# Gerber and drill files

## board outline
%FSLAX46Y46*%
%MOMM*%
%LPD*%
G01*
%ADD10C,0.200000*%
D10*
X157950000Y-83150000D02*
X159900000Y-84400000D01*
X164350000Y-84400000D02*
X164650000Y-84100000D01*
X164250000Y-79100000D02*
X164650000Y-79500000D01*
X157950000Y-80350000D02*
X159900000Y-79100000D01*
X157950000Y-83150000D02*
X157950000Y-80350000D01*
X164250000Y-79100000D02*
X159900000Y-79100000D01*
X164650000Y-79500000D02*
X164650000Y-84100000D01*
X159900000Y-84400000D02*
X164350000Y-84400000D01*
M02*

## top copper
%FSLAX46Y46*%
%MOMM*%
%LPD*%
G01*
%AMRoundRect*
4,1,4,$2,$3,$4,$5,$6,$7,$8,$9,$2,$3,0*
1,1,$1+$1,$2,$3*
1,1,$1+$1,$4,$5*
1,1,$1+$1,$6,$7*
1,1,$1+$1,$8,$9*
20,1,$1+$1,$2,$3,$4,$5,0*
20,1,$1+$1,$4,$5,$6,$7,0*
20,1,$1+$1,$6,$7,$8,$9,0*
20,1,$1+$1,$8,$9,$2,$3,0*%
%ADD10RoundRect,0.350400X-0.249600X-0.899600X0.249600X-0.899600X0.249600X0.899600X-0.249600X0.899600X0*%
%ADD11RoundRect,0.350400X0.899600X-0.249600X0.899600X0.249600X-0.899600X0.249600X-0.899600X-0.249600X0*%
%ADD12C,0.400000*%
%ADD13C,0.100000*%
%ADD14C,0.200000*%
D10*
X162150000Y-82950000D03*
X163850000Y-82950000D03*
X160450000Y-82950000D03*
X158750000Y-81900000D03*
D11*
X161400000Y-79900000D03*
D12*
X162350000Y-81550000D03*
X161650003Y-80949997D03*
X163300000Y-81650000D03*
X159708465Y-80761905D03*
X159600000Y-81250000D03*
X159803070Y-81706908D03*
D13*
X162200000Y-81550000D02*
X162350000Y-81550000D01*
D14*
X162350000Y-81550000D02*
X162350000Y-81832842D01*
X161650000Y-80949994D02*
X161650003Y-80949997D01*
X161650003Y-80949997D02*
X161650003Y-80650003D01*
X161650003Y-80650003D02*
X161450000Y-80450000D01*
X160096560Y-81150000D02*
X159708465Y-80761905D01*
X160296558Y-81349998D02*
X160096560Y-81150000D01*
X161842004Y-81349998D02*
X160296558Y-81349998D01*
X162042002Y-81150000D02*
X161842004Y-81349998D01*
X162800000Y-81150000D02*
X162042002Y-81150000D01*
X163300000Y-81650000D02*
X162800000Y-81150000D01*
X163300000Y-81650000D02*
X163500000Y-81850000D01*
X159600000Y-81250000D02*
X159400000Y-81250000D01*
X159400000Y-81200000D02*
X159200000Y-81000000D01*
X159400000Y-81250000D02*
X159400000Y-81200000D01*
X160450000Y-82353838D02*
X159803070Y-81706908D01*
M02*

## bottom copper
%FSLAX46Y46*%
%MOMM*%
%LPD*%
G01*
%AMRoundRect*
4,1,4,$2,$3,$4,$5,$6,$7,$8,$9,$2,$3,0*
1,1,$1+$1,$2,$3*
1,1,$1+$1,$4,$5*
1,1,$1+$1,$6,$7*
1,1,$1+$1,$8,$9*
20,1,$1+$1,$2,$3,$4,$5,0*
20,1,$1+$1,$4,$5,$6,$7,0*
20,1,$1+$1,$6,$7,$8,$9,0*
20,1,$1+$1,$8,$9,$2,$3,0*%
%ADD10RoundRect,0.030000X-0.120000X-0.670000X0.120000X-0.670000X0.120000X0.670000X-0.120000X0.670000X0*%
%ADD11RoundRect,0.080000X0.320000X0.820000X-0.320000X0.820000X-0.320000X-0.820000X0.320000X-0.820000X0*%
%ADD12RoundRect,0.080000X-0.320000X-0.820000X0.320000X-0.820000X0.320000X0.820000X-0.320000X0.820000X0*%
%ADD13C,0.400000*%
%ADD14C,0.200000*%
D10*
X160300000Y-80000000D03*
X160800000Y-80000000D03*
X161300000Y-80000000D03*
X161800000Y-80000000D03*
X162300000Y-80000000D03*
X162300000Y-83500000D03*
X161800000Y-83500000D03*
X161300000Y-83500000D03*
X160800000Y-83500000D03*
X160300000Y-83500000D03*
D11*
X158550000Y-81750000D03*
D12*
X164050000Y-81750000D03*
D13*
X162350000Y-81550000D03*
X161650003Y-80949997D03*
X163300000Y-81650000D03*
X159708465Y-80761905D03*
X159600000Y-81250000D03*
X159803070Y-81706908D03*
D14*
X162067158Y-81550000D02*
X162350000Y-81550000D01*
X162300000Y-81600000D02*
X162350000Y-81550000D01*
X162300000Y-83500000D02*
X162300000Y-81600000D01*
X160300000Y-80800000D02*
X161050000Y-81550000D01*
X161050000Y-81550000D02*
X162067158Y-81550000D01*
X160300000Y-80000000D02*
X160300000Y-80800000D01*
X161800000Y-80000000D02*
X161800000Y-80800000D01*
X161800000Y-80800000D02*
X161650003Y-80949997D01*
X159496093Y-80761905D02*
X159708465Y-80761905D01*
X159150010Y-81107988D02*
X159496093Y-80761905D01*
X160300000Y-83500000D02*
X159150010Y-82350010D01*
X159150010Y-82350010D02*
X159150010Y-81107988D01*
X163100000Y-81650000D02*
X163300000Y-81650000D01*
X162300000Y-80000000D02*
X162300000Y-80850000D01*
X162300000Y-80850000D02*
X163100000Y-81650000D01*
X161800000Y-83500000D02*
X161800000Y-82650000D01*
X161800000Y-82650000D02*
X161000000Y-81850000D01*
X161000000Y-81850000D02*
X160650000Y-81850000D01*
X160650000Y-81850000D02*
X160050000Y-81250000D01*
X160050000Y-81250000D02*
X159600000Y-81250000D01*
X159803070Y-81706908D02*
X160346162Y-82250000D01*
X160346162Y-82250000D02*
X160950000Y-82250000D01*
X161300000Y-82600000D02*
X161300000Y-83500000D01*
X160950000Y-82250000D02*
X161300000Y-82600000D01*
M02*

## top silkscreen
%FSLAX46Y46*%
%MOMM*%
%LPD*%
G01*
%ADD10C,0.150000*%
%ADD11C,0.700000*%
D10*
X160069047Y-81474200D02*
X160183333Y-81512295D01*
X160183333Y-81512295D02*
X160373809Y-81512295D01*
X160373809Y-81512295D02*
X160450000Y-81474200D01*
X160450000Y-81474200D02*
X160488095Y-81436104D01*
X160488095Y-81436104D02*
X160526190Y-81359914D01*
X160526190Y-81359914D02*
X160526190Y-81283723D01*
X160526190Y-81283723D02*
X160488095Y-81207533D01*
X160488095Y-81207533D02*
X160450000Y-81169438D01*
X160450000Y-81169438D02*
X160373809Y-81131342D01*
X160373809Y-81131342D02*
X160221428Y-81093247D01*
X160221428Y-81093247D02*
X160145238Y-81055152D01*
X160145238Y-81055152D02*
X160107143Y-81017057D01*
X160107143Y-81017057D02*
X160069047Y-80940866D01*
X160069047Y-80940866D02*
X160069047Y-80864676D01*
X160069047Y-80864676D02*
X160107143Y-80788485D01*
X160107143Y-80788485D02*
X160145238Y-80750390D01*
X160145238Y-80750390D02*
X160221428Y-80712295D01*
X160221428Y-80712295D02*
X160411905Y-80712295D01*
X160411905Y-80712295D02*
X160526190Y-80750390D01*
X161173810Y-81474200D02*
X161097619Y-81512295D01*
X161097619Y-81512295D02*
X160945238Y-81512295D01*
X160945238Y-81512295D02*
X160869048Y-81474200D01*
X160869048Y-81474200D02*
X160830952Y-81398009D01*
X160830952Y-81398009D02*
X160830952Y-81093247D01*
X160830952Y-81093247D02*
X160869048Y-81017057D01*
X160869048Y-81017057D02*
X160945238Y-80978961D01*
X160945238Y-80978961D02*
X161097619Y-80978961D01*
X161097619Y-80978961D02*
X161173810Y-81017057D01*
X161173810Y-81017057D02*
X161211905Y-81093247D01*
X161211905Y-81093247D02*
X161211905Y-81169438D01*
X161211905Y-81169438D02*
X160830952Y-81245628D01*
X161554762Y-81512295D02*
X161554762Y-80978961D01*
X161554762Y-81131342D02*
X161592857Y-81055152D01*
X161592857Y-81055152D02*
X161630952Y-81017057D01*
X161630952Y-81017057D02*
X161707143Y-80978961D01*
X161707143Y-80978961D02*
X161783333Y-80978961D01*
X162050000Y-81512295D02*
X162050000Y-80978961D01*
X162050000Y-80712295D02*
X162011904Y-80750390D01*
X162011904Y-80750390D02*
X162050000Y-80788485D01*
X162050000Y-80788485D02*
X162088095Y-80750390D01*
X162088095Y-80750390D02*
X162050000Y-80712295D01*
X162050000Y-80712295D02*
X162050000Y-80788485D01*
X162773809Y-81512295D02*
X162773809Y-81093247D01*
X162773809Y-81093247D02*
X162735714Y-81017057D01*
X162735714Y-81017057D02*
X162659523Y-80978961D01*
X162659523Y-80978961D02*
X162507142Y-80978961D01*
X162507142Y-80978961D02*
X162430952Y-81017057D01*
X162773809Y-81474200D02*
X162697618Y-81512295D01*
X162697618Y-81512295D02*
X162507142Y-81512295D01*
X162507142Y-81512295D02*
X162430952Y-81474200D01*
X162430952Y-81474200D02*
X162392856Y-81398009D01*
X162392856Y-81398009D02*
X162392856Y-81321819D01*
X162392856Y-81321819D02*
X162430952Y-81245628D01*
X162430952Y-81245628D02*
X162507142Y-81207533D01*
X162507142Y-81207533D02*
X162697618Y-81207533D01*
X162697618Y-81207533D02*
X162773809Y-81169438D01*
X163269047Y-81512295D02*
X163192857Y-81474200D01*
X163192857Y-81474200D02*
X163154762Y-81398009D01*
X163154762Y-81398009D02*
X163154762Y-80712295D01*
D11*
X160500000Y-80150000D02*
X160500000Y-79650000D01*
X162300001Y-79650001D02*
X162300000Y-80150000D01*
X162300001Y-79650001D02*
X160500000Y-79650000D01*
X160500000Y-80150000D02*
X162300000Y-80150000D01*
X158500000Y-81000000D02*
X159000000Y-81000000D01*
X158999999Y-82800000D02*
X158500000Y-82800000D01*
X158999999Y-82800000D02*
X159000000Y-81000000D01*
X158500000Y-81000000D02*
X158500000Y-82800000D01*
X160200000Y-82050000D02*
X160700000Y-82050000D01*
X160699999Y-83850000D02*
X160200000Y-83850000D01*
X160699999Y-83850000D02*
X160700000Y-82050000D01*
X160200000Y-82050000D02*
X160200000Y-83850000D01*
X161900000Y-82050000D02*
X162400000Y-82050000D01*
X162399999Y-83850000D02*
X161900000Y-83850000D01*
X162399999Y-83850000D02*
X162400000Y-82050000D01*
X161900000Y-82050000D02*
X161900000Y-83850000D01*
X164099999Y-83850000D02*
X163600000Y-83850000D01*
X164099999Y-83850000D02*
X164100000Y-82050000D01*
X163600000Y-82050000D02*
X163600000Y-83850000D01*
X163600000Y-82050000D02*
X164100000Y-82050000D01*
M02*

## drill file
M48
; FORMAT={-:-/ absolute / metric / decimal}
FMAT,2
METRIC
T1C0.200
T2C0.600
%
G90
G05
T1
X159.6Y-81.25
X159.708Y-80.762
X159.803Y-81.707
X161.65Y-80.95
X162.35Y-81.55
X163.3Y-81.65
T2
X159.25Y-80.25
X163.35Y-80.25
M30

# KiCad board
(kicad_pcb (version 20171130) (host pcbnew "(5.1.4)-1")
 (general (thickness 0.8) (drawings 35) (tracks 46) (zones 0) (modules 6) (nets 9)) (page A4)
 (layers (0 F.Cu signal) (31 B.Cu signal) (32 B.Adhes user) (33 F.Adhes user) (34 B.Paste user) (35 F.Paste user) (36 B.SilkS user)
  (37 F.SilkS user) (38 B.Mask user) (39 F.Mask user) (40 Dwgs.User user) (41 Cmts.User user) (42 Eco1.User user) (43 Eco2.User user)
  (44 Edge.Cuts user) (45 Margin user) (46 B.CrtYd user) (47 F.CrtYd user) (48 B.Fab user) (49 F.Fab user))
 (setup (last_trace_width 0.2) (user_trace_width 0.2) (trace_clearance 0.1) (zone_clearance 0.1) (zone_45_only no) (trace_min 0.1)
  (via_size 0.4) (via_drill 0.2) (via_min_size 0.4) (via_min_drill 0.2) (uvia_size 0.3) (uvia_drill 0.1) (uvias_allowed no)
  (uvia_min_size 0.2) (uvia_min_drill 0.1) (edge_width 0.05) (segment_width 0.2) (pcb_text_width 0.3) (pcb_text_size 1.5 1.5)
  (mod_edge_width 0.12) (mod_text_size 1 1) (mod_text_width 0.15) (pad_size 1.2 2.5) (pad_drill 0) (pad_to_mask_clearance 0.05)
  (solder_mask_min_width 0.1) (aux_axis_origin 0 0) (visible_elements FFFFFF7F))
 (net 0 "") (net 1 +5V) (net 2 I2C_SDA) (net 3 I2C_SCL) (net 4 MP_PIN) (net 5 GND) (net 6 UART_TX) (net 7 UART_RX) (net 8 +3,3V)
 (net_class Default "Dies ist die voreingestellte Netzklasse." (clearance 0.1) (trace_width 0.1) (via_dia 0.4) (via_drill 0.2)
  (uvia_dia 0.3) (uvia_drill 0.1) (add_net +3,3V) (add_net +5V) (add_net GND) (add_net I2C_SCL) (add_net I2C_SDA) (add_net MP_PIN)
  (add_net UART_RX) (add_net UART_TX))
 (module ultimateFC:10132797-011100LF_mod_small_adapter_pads (layer B.Cu) (at 161.3 81.75 180)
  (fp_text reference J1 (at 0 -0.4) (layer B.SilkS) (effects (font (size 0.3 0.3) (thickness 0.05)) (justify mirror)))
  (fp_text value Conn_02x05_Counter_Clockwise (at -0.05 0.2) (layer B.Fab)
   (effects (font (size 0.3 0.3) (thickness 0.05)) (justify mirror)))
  (pad 1 smd roundrect (at 1 1.75) (size 0.3 1.4) (layers B.Cu B.Paste B.Mask) (roundrect_rratio 0.1) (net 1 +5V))
  (pad 2 smd roundrect (at 0.5 1.75) (size 0.3 1.4) (layers B.Cu B.Paste B.Mask) (roundrect_rratio 0.1) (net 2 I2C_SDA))
  (pad 3 smd roundrect (at 0 1.75) (size 0.3 1.4) (layers B.Cu B.Paste B.Mask) (roundrect_rratio 0.1) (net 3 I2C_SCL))
  (pad 4 smd roundrect (at -0.5 1.75) (size 0.3 1.4) (layers B.Cu B.Paste B.Mask) (roundrect_rratio 0.1) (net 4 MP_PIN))
  (pad 5 smd roundrect (at -1 1.75) (size 0.3 1.4) (layers B.Cu B.Paste B.Mask) (roundrect_rratio 0.1) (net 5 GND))
  (pad 6 smd roundrect (at -1 -1.75) (size 0.3 1.4) (layers B.Cu B.Paste B.Mask) (roundrect_rratio 0.1) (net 1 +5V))
  (pad 7 smd roundrect (at -0.5 -1.75) (size 0.3 1.4) (layers B.Cu B.Paste B.Mask) (roundrect_rratio 0.1) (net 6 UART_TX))
  (pad 8 smd roundrect (at 0 -1.75) (size 0.3 1.4) (layers B.Cu B.Paste B.Mask) (roundrect_rratio 0.1) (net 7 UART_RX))
  (pad 9 smd roundrect (at 0.5 -1.75) (size 0.3 1.4) (layers B.Cu B.Paste B.Mask) (roundrect_rratio 0.1) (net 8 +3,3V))
  (pad 10 smd roundrect (at 1 -1.75) (size 0.3 1.4) (layers B.Cu B.Paste B.Mask) (roundrect_rratio 0.1) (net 5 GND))
  (pad "" smd roundrect (at 2.75 0 180) (size 0.8 1.8) (layers B.Cu B.Paste B.Mask) (roundrect_rratio 0.1))
  (pad "" smd roundrect (at -2.75 0) (size 0.8 1.8) (layers B.Cu B.Paste B.Mask) (roundrect_rratio 0.1))
  (pad "" np_thru_hole circle (at 2.05 1.5 180) (size 0.6 0.6) (drill 0.6) (layers *.Cu *.Mask) (solder_mask_margin -0.001))
  (pad "" np_thru_hole circle (at -2.05 1.5 180) (size 0.6 0.6) (drill 0.6) (layers *.Cu *.Mask) (solder_mask_margin -0.001)))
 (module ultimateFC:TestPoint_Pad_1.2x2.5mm (layer F.Cu) (at 162.15 82.95)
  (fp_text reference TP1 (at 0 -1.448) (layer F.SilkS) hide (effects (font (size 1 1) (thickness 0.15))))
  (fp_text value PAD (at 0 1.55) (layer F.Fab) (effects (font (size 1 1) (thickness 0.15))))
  (pad 1 smd roundrect (at 0 0) (size 1.2 2.5) (layers F.Cu F.Mask) (roundrect_rratio 0.292) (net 1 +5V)))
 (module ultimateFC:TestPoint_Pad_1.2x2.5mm (layer F.Cu) (at 163.85 82.95)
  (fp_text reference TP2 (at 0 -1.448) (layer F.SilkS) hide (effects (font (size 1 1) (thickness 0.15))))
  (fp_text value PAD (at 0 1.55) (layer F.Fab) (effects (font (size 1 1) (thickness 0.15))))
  (pad 1 smd roundrect (at 0 0) (size 1.2 2.5) (layers F.Cu F.Mask) (roundrect_rratio 0.292) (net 5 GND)))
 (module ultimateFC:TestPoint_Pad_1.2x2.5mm (layer F.Cu) (at 160.45 82.95)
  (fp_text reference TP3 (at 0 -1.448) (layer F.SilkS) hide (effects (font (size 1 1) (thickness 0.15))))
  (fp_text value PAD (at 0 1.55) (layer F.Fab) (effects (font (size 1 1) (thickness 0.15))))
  (pad 1 smd roundrect (at 0 0) (size 1.2 2.5) (layers F.Cu F.Mask) (roundrect_rratio 0.292) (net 7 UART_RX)))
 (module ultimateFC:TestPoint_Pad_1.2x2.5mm (layer F.Cu) (at 158.75 81.9)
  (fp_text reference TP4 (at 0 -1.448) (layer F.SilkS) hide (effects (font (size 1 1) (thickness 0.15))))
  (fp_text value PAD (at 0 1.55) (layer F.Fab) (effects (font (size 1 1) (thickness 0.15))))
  (pad 1 smd roundrect (at 0 0) (size 1.2 2.5) (layers F.Cu F.Mask) (roundrect_rratio 0.292) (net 6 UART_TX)))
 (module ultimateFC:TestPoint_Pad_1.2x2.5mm (layer F.Cu) (at 161.4 79.9 90)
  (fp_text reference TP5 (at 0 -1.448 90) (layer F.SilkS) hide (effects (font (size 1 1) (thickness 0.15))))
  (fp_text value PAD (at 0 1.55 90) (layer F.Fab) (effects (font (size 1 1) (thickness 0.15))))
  (pad 1 smd roundrect (at 0 0 90) (size 1.2 2.5) (layers F.Cu F.Mask) (roundrect_rratio 0.292) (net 4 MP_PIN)))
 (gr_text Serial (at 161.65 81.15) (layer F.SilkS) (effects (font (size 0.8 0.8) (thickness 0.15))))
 (gr_line (start 160.5 80.15) (end 160.5 79.65) (layer F.SilkS) (width 0.7))
 (gr_line (start 162.300001 79.650001) (end 162.3 80.15) (layer F.SilkS) (width 0.7))
 (gr_line (start 162.300001 79.650001) (end 160.5 79.65) (layer F.SilkS) (width 0.7))
 (gr_line (start 160.5 80.15) (end 162.3 80.15) (layer F.SilkS) (width 0.7))
 (gr_line (start 158.5 81) (end 159 81) (layer F.SilkS) (width 0.7))
 (gr_line (start 158.999999 82.8) (end 158.5 82.8) (layer F.SilkS) (width 0.7))
 (gr_line (start 158.999999 82.8) (end 159 81) (layer F.SilkS) (width 0.7))
 (gr_line (start 158.5 81) (end 158.5 82.8) (layer F.SilkS) (width 0.7))
 (gr_line (start 160.2 82.05) (end 160.7 82.05) (layer F.SilkS) (width 0.7))
 (gr_line (start 160.699999 83.85) (end 160.2 83.85) (layer F.SilkS) (width 0.7))
 (gr_line (start 160.699999 83.85) (end 160.7 82.05) (layer F.SilkS) (width 0.7))
 (gr_line (start 160.2 82.05) (end 160.2 83.85) (layer F.SilkS) (width 0.7))
 (gr_line (start 161.9 82.05) (end 162.4 82.05) (layer F.SilkS) (width 0.7))
 (gr_line (start 162.399999 83.85) (end 161.9 83.85) (layer F.SilkS) (width 0.7))
 (gr_line (start 162.399999 83.85) (end 162.4 82.05) (layer F.SilkS) (width 0.7))
 (gr_line (start 161.9 82.05) (end 161.9 83.85) (layer F.SilkS) (width 0.7))
 (gr_line (start 164.099999 83.85) (end 163.6 83.85) (layer F.SilkS) (width 0.7))
 (gr_line (start 164.099999 83.85) (end 164.1 82.05) (layer F.SilkS) (width 0.7))
 (gr_line (start 163.6 82.05) (end 163.6 83.85) (layer F.SilkS) (width 0.7))
 (gr_line (start 163.6 82.05) (end 164.1 82.05) (layer F.SilkS) (width 0.7))
 (gr_line (start 157.95 83.15) (end 159.9 84.4) (layer Edge.Cuts) (width 0.2))
 (gr_line (start 164.35 84.4) (end 164.65 84.1) (layer Edge.Cuts) (width 0.2))
 (gr_line (start 164.25 79.1) (end 164.65 79.5) (layer Edge.Cuts) (width 0.2))
 (gr_line (start 157.95 80.35) (end 159.9 79.1) (layer Edge.Cuts) (width 0.2))
 (gr_line (start 157.95 83.15) (end 157.95 80.35) (layer Edge.Cuts) (width 0.2))
 (gr_line (start 164.25 79.1) (end 159.9 79.1) (layer Edge.Cuts) (width 0.2))
 (gr_line (start 164.65 79.5) (end 164.65 84.1) (layer Edge.Cuts) (width 0.2))
 (gr_line (start 159.9 84.4) (end 164.35 84.4) (layer Edge.Cuts) (width 0.2))
 (segment (start 162.067158 81.55) (end 162.35 81.55) (width 0.2) (layer B.Cu) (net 1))
 (segment (start 162.3 81.6) (end 162.35 81.55) (width 0.2) (layer B.Cu) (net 1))
 (segment (start 162.3 83.5) (end 162.3 81.6) (width 0.2) (layer B.Cu) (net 1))
 (segment (start 162.2 81.55) (end 162.35 81.55) (width 0.1) (layer F.Cu) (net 1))
 (segment (start 160.3 80.8) (end 161.05 81.55) (width 0.2) (layer B.Cu) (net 1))
 (segment (start 161.05 81.55) (end 162.067158 81.55) (width 0.2) (layer B.Cu) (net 1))
 (segment (start 160.3 80) (end 160.3 80.8) (width 0.2) (layer B.Cu) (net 1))
 (via (at 162.35 81.55) (size 0.4) (drill 0.2) (layers F.Cu B.Cu) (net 1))
 (segment (start 162.35 81.55) (end 162.35 81.832842) (width 0.2) (layer F.Cu) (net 1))
 (via (at 161.650003 80.949997) (size 0.4) (drill 0.2) (layers F.Cu B.Cu) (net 4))
 (segment (start 161.8 80) (end 161.8 80.8) (width 0.2) (layer B.Cu) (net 4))
 (segment (start 161.8 80.8) (end 161.650003 80.949997) (width 0.2) (layer B.Cu) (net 4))
 (segment (start 161.65 80.949994) (end 161.650003 80.949997) (width 0.2) (layer F.Cu) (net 4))
 (segment (start 161.650003 80.949997) (end 161.650003 80.650003) (width 0.2) (layer F.Cu) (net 4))
 (segment (start 161.650003 80.650003) (end 161.45 80.45) (width 0.2) (layer F.Cu) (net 4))
 (via (at 163.3 81.65) (size 0.4) (drill 0.2) (layers F.Cu B.Cu) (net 5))
 (via (at 159.708465 80.761905) (size 0.4) (drill 0.2) (layers F.Cu B.Cu) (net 5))
 (segment (start 159.496093 80.761905) (end 159.708465 80.761905) (width 0.2) (layer B.Cu) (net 5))
 (segment (start 159.15001 81.107988) (end 159.496093 80.761905) (width 0.2) (layer B.Cu) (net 5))
 (segment (start 160.3 83.5) (end 159.15001 82.35001) (width 0.2) (layer B.Cu) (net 5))
 (segment (start 159.15001 82.35001) (end 159.15001 81.107988) (width 0.2) (layer B.Cu) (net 5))
 (segment (start 163.1 81.65) (end 163.3 81.65) (width 0.2) (layer B.Cu) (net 5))
 (segment (start 162.3 80) (end 162.3 80.85) (width 0.2) (layer B.Cu) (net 5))
 (segment (start 162.3 80.85) (end 163.1 81.65) (width 0.2) (layer B.Cu) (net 5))
 (segment (start 160.09656 81.15) (end 159.708465 80.761905) (width 0.2) (layer F.Cu) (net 5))
 (segment (start 160.296558 81.349998) (end 160.09656 81.15) (width 0.2) (layer F.Cu) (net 5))
 (segment (start 161.842004 81.349998) (end 160.296558 81.349998) (width 0.2) (layer F.Cu) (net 5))
 (segment (start 162.042002 81.15) (end 161.842004 81.349998) (width 0.2) (layer F.Cu) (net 5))
 (segment (start 162.8 81.15) (end 162.042002 81.15) (width 0.2) (layer F.Cu) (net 5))
 (segment (start 163.3 81.65) (end 162.8 81.15) (width 0.2) (layer F.Cu) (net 5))
 (segment (start 163.3 81.65) (end 163.5 81.85) (width 0.2) (layer F.Cu) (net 5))
 (segment (start 161.8 83.5) (end 161.8 82.65) (width 0.2) (layer B.Cu) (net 6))
 (segment (start 161.8 82.65) (end 161 81.85) (width 0.2) (layer B.Cu) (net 6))
 (segment (start 161 81.85) (end 160.65 81.85) (width 0.2) (layer B.Cu) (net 6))
 (via (at 159.6 81.25) (size 0.4) (drill 0.2) (layers F.Cu B.Cu) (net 6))
 (segment (start 160.65 81.85) (end 160.05 81.25) (width 0.2) (layer B.Cu) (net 6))
 (segment (start 160.05 81.25) (end 159.6 81.25) (width 0.2) (layer B.Cu) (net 6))
 (segment (start 159.6 81.25) (end 159.4 81.25) (width 0.2) (layer F.Cu) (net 6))
 (segment (start 159.4 81.2) (end 159.2 81) (width 0.2) (layer F.Cu) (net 6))
 (segment (start 159.4 81.25) (end 159.4 81.2) (width 0.2) (layer F.Cu) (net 6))
 (via (at 159.80307 81.706908) (size 0.4) (drill 0.2) (layers F.Cu B.Cu) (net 7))
 (segment (start 160.45 82.353838) (end 159.80307 81.706908) (width 0.2) (layer F.Cu) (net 7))
 (segment (start 159.80307 81.706908) (end 160.346162 82.25) (width 0.2) (layer B.Cu) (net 7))
 (segment (start 160.346162 82.25) (end 160.95 82.25) (width 0.2) (layer B.Cu) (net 7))
 (segment (start 161.3 82.6) (end 161.3 83.5) (width 0.2) (layer B.Cu) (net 7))
 (segment (start 160.95 82.25) (end 161.3 82.6) (width 0.2) (layer B.Cu) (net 7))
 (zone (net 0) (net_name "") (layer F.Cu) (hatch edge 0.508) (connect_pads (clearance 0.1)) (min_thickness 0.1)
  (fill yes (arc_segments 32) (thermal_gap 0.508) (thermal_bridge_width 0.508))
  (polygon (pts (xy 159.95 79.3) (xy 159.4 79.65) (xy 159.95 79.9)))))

